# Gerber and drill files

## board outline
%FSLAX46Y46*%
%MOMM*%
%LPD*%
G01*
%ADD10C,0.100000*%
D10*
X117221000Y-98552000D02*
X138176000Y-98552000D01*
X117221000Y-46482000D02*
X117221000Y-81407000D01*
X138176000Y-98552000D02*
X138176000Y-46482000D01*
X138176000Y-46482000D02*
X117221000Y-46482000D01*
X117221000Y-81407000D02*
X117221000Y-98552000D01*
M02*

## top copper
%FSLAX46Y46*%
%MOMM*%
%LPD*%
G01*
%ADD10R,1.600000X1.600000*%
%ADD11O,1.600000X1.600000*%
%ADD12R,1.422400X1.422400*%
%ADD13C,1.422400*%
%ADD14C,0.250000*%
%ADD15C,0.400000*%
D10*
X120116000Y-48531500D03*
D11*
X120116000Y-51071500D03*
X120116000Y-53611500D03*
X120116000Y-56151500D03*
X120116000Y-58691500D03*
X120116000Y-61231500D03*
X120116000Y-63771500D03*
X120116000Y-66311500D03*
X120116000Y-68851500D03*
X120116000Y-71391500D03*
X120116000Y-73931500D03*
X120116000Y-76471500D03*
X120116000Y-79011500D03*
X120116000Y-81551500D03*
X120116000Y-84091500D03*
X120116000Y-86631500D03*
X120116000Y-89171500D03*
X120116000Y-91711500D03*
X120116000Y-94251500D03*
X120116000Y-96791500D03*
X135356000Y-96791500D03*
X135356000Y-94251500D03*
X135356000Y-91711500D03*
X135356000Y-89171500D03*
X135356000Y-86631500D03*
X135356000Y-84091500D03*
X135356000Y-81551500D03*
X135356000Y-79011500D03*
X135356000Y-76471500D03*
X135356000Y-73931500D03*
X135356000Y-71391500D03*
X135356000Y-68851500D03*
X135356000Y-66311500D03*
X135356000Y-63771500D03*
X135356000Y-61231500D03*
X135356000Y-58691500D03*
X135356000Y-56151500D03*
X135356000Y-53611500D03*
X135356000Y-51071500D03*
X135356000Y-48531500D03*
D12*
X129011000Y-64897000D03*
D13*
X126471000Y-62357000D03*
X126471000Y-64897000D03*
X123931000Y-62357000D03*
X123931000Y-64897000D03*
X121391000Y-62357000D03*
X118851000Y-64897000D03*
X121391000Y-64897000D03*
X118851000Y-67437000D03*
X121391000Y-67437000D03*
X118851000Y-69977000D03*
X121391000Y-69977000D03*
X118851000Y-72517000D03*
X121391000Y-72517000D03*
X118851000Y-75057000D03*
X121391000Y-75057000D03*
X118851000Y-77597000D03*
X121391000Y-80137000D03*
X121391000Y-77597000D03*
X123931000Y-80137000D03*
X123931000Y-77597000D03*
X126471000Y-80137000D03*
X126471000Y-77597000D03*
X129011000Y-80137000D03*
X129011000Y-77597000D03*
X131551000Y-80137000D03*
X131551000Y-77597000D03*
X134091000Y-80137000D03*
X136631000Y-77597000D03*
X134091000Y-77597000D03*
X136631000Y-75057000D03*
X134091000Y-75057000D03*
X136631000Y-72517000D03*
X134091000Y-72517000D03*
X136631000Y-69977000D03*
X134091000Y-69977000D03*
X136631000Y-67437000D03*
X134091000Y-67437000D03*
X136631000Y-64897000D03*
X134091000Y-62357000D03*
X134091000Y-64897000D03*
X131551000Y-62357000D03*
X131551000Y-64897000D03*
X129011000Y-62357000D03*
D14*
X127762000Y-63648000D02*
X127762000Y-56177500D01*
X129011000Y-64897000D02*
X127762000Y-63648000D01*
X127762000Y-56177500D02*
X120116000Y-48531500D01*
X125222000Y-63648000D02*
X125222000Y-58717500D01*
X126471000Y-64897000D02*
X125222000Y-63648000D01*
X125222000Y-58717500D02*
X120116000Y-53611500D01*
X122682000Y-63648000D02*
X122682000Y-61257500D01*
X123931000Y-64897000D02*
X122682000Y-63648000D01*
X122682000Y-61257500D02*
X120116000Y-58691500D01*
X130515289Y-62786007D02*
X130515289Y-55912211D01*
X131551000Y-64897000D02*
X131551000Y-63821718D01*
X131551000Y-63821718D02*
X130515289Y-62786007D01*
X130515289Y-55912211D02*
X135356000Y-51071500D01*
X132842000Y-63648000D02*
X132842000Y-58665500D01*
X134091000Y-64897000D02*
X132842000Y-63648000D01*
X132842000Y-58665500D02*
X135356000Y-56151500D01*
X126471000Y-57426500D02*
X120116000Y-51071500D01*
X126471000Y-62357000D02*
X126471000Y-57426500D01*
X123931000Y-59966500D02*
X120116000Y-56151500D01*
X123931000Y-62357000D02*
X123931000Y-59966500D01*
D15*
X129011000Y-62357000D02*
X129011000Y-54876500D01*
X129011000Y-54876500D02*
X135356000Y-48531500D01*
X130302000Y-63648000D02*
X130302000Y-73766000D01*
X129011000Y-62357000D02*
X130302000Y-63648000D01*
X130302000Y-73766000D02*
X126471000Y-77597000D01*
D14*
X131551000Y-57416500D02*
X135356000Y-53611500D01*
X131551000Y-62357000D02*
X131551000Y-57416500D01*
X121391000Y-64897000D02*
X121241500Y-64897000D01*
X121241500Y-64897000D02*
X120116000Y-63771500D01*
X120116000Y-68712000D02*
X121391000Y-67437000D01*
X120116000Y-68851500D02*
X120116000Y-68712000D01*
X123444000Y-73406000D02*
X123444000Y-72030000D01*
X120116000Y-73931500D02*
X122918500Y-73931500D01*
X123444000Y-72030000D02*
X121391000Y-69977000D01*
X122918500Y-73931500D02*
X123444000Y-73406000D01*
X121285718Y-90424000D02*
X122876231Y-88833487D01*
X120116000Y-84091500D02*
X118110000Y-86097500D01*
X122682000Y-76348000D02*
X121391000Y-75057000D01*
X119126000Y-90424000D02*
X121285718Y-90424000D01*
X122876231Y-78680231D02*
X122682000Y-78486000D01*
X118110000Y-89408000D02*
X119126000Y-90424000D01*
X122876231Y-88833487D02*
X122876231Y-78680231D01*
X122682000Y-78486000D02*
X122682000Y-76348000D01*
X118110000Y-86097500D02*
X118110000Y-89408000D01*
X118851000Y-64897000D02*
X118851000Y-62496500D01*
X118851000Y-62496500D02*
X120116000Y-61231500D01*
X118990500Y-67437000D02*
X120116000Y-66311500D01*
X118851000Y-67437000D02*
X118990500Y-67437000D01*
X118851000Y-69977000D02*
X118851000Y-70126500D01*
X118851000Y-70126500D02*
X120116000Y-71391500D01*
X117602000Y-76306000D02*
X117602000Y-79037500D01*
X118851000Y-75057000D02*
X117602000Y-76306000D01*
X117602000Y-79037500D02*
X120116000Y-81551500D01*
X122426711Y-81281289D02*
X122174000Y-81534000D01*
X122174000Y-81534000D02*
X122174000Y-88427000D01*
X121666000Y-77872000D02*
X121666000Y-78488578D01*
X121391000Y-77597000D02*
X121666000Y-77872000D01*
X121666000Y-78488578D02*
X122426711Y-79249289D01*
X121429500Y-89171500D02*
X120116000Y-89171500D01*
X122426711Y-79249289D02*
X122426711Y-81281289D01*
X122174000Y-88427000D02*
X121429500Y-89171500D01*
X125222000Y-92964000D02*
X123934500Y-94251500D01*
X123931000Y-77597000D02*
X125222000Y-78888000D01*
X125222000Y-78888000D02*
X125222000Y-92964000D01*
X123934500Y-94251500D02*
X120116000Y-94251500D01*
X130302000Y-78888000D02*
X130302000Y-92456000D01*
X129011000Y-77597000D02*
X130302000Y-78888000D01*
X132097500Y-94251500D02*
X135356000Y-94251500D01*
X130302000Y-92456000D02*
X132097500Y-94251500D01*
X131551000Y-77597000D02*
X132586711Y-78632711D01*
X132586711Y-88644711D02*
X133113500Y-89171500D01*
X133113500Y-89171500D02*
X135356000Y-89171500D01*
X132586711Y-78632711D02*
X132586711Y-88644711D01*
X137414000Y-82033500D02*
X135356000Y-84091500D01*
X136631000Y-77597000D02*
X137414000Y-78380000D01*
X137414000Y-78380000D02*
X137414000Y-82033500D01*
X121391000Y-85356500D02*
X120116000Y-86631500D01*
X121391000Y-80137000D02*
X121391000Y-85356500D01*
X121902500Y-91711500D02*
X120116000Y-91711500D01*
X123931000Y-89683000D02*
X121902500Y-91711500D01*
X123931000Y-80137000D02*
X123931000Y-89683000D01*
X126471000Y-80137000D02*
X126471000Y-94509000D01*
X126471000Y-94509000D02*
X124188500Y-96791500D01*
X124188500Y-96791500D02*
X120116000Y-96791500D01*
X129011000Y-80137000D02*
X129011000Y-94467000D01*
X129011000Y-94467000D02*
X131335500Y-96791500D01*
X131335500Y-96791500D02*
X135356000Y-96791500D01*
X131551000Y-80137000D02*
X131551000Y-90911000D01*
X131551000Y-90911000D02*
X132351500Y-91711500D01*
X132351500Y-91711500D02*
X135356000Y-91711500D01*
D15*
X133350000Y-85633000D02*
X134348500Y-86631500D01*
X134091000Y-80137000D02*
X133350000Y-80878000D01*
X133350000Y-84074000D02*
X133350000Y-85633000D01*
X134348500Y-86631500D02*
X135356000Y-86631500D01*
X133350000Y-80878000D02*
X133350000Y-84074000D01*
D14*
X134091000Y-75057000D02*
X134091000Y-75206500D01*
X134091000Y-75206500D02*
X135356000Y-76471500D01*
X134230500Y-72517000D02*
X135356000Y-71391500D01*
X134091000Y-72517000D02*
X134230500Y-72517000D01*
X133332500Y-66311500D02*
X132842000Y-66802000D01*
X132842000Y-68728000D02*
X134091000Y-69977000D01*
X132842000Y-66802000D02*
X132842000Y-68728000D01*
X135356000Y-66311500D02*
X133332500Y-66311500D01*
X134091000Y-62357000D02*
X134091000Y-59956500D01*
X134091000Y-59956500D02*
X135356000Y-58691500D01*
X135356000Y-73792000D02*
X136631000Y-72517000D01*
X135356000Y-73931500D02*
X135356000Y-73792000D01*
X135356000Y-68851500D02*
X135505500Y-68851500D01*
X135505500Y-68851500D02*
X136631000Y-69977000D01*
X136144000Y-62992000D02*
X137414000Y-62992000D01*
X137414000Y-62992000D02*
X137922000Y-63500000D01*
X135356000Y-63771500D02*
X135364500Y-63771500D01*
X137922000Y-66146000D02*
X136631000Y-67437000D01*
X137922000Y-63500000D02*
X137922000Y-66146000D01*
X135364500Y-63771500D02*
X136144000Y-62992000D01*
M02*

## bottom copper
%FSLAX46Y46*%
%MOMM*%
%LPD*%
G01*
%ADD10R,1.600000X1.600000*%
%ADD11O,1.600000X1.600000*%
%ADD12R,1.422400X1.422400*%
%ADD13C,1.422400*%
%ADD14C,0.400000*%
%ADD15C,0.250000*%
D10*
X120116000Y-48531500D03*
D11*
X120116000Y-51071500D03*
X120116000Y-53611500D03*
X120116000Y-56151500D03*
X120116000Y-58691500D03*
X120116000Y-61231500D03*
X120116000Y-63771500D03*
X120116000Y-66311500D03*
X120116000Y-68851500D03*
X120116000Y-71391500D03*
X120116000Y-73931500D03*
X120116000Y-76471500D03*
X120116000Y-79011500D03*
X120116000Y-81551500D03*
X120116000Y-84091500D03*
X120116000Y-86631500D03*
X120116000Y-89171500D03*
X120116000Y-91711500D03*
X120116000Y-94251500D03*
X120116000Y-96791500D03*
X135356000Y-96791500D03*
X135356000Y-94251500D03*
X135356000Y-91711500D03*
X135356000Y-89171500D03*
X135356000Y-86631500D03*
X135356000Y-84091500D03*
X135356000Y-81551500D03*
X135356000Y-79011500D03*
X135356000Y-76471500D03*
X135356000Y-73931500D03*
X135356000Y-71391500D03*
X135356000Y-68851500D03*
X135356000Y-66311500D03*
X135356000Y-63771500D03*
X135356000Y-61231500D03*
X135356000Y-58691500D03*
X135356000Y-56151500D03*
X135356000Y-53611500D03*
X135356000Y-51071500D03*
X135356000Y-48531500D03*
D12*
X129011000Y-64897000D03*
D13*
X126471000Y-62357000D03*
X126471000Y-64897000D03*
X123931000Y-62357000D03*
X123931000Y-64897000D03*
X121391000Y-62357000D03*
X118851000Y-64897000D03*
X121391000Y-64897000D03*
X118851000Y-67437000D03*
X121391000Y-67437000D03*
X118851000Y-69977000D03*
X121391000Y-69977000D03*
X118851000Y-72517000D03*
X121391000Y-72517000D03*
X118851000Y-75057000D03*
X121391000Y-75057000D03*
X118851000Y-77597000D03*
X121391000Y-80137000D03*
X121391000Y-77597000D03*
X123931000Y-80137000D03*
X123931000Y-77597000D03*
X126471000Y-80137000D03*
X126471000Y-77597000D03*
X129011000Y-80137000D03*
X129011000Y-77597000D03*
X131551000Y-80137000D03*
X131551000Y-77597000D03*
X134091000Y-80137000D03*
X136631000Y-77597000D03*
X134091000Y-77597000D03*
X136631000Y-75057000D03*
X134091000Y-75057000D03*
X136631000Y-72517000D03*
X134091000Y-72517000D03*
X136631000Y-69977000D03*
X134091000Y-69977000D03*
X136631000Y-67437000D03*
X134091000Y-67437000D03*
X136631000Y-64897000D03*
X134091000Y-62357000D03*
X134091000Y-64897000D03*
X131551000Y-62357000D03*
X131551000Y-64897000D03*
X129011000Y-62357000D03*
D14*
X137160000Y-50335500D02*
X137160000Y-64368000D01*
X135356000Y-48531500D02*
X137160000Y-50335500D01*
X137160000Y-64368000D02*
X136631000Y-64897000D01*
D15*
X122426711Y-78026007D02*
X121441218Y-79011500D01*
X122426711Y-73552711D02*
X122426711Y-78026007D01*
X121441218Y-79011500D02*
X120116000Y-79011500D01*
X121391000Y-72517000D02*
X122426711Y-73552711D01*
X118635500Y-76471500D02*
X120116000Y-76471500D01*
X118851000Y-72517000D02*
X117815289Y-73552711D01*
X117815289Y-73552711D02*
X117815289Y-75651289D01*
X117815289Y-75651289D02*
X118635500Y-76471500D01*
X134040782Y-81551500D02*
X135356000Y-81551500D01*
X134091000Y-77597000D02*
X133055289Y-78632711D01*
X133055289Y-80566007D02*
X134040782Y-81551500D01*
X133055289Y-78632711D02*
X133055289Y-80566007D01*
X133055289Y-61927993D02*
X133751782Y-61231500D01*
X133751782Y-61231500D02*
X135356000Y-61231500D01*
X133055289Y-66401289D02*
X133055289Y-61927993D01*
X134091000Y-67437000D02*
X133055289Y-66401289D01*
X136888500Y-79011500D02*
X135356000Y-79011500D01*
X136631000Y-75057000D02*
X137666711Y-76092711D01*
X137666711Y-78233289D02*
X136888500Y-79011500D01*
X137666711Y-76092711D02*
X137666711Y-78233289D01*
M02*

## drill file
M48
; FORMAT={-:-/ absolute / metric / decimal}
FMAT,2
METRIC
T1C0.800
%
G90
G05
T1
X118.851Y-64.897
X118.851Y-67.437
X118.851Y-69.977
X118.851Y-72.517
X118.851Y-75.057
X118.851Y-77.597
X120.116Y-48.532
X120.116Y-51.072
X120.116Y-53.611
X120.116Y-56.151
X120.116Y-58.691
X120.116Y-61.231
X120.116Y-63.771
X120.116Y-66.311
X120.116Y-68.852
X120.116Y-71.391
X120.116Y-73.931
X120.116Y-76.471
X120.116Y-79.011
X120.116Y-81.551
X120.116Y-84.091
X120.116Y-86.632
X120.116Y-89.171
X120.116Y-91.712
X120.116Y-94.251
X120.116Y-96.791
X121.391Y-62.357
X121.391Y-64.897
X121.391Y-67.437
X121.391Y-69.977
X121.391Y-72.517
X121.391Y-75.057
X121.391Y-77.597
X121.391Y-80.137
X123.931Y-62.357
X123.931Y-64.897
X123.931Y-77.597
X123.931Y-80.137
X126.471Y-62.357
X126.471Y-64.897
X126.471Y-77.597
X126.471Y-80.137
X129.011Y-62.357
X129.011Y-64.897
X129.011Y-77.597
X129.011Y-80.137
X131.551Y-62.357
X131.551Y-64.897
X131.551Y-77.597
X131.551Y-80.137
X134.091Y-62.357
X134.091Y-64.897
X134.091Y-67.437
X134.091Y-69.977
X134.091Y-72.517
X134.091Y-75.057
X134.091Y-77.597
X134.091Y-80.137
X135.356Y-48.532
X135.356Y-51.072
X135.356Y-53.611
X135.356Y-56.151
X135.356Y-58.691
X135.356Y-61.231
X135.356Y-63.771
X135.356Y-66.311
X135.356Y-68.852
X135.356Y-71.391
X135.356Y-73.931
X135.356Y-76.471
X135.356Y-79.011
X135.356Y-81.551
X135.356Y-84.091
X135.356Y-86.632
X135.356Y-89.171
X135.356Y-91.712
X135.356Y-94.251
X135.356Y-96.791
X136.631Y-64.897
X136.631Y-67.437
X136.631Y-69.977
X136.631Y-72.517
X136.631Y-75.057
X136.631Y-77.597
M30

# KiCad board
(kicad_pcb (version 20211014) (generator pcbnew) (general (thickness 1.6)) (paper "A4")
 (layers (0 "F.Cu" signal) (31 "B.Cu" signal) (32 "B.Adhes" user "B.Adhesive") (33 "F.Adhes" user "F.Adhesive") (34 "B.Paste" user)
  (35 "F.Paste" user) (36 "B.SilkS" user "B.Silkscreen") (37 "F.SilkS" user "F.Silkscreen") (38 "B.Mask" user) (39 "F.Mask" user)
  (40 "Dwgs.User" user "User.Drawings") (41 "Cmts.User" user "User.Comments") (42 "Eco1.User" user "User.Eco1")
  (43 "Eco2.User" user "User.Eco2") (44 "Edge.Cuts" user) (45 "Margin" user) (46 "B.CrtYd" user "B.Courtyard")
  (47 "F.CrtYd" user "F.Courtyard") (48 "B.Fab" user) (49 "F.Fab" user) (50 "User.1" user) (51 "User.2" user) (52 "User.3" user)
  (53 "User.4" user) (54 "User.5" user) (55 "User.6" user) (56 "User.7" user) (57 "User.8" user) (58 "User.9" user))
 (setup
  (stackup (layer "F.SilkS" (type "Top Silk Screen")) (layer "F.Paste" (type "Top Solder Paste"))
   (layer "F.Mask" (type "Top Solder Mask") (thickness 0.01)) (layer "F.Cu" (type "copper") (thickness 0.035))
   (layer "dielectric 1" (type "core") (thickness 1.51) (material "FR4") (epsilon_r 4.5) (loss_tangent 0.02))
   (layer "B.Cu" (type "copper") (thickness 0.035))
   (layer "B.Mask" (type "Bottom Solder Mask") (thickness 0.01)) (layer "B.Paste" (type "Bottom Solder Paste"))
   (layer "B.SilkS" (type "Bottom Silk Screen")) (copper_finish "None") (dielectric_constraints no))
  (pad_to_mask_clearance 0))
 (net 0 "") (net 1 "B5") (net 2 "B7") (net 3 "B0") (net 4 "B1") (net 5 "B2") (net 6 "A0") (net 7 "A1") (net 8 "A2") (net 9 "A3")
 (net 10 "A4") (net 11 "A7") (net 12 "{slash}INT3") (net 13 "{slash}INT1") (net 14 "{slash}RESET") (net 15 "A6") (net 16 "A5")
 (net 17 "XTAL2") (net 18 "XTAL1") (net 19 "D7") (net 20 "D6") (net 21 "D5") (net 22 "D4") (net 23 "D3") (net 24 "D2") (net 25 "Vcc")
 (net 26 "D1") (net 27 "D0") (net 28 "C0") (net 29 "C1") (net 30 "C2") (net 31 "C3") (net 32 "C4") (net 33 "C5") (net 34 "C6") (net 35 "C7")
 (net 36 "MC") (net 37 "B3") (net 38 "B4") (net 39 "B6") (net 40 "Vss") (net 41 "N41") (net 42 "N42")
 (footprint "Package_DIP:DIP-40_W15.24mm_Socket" (layer "F.Cu") (at 120.116 48.5315)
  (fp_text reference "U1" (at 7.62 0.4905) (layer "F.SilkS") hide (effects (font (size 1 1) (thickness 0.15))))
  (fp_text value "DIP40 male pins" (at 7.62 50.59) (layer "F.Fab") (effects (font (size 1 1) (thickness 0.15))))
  (pad "1" thru_hole rect locked (at 0 0) (size 1.6 1.6) (drill 0.8) (layers *.Cu *.Mask) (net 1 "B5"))
  (pad "2" thru_hole oval locked (at 0 2.54) (size 1.6 1.6) (drill 0.8) (layers *.Cu *.Mask) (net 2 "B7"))
  (pad "3" thru_hole oval locked (at 0 5.08) (size 1.6 1.6) (drill 0.8) (layers *.Cu *.Mask) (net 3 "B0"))
  (pad "4" thru_hole oval locked (at 0 7.62) (size 1.6 1.6) (drill 0.8) (layers *.Cu *.Mask) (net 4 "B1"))
  (pad "5" thru_hole oval locked (at 0 10.16) (size 1.6 1.6) (drill 0.8) (layers *.Cu *.Mask) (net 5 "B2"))
  (pad "6" thru_hole oval locked (at 0 12.7) (size 1.6 1.6) (drill 0.8) (layers *.Cu *.Mask) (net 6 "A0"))
  (pad "7" thru_hole oval locked (at 0 15.24) (size 1.6 1.6) (drill 0.8) (layers *.Cu *.Mask) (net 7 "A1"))
  (pad "8" thru_hole oval locked (at 0 17.78) (size 1.6 1.6) (drill 0.8) (layers *.Cu *.Mask) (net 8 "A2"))
  (pad "9" thru_hole oval locked (at 0 20.32) (size 1.6 1.6) (drill 0.8) (layers *.Cu *.Mask) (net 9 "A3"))
  (pad "10" thru_hole oval locked (at 0 22.86) (size 1.6 1.6) (drill 0.8) (layers *.Cu *.Mask) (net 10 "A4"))
  (pad "11" thru_hole oval locked (at 0 25.4) (size 1.6 1.6) (drill 0.8) (layers *.Cu *.Mask) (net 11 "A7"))
  (pad "12" thru_hole oval locked (at 0 27.94) (size 1.6 1.6) (drill 0.8) (layers *.Cu *.Mask) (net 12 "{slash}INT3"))
  (pad "13" thru_hole oval locked (at 0 30.48) (size 1.6 1.6) (drill 0.8) (layers *.Cu *.Mask) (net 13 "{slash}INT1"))
  (pad "14" thru_hole oval locked (at 0 33.02) (size 1.6 1.6) (drill 0.8) (layers *.Cu *.Mask) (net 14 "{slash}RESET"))
  (pad "15" thru_hole oval locked (at 0 35.56) (size 1.6 1.6) (drill 0.8) (layers *.Cu *.Mask) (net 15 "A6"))
  (pad "16" thru_hole oval locked (at 0 38.1) (size 1.6 1.6) (drill 0.8) (layers *.Cu *.Mask) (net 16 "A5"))
  (pad "17" thru_hole oval locked (at 0 40.64) (size 1.6 1.6) (drill 0.8) (layers *.Cu *.Mask) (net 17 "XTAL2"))
  (pad "18" thru_hole oval locked (at 0 43.18) (size 1.6 1.6) (drill 0.8) (layers *.Cu *.Mask) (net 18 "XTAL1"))
  (pad "19" thru_hole oval locked (at 0 45.72) (size 1.6 1.6) (drill 0.8) (layers *.Cu *.Mask) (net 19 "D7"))
  (pad "20" thru_hole oval locked (at 0 48.26) (size 1.6 1.6) (drill 0.8) (layers *.Cu *.Mask) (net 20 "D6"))
  (pad "21" thru_hole oval locked (at 15.24 48.26) (size 1.6 1.6) (drill 0.8) (layers *.Cu *.Mask) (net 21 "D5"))
  (pad "22" thru_hole oval locked (at 15.24 45.72) (size 1.6 1.6) (drill 0.8) (layers *.Cu *.Mask) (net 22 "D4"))
  (pad "23" thru_hole oval locked (at 15.24 43.18) (size 1.6 1.6) (drill 0.8) (layers *.Cu *.Mask) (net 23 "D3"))
  (pad "24" thru_hole oval locked (at 15.24 40.64) (size 1.6 1.6) (drill 0.8) (layers *.Cu *.Mask) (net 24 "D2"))
  (pad "25" thru_hole oval locked (at 15.24 38.1) (size 1.6 1.6) (drill 0.8) (layers *.Cu *.Mask) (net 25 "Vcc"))
  (pad "26" thru_hole oval locked (at 15.24 35.56) (size 1.6 1.6) (drill 0.8) (layers *.Cu *.Mask) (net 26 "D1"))
  (pad "27" thru_hole oval locked (at 15.24 33.02) (size 1.6 1.6) (drill 0.8) (layers *.Cu *.Mask) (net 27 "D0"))
  (pad "28" thru_hole oval locked (at 15.24 30.48) (size 1.6 1.6) (drill 0.8) (layers *.Cu *.Mask) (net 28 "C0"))
  (pad "29" thru_hole oval locked (at 15.24 27.94) (size 1.6 1.6) (drill 0.8) (layers *.Cu *.Mask) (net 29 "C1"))
  (pad "30" thru_hole oval locked (at 15.24 25.4) (size 1.6 1.6) (drill 0.8) (layers *.Cu *.Mask) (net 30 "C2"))
  (pad "31" thru_hole oval locked (at 15.24 22.86) (size 1.6 1.6) (drill 0.8) (layers *.Cu *.Mask) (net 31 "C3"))
  (pad "32" thru_hole oval locked (at 15.24 20.32) (size 1.6 1.6) (drill 0.8) (layers *.Cu *.Mask) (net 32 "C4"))
  (pad "33" thru_hole oval locked (at 15.24 17.78) (size 1.6 1.6) (drill 0.8) (layers *.Cu *.Mask) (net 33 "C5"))
  (pad "34" thru_hole oval locked (at 15.24 15.24) (size 1.6 1.6) (drill 0.8) (layers *.Cu *.Mask) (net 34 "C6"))
  (pad "35" thru_hole oval locked (at 15.24 12.7) (size 1.6 1.6) (drill 0.8) (layers *.Cu *.Mask) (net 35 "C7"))
  (pad "36" thru_hole oval locked (at 15.24 10.16) (size 1.6 1.6) (drill 0.8) (layers *.Cu *.Mask) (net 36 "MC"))
  (pad "37" thru_hole oval locked (at 15.24 7.62) (size 1.6 1.6) (drill 0.8) (layers *.Cu *.Mask) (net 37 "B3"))
  (pad "38" thru_hole oval locked (at 15.24 5.08) (size 1.6 1.6) (drill 0.8) (layers *.Cu *.Mask) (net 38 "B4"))
  (pad "39" thru_hole oval locked (at 15.24 2.54) (size 1.6 1.6) (drill 0.8) (layers *.Cu *.Mask) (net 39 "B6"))
  (pad "40" thru_hole oval locked (at 15.24 0) (size 1.6 1.6) (drill 0.8) (layers *.Cu *.Mask) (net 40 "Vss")))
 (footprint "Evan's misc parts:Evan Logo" (layer "F.Cu") (at 127.381 91.567)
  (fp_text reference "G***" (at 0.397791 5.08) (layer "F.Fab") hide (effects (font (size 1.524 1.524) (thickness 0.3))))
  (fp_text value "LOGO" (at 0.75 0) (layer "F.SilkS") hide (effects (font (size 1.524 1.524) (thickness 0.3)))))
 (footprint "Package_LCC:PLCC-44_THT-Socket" (layer "F.Cu") (at 129.011 64.897)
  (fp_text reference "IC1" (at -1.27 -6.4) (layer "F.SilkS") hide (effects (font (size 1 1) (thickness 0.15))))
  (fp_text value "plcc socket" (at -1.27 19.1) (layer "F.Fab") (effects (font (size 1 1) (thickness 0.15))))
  (pad "1" thru_hole rect locked (at 0 0) (size 1.4224 1.4224) (drill 0.8) (layers *.Cu *.Mask) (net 1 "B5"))
  (pad "2" thru_hole circle locked (at -2.54 -2.54) (size 1.4224 1.4224) (drill 0.8) (layers *.Cu *.Mask) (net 2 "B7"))
  (pad "3" thru_hole circle locked (at -2.54 0) (size 1.4224 1.4224) (drill 0.8) (layers *.Cu *.Mask) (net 3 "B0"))
  (pad "4" thru_hole circle locked (at -5.08 -2.54) (size 1.4224 1.4224) (drill 0.8) (layers *.Cu *.Mask) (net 4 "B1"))
  (pad "5" thru_hole circle locked (at -5.08 0) (size 1.4224 1.4224) (drill 0.8) (layers *.Cu *.Mask) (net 5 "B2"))
  (pad "6" thru_hole circle locked (at -7.62 -2.54) (size 1.4224 1.4224) (drill 0.8) (layers *.Cu *.Mask) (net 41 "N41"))
  (pad "7" thru_hole circle locked (at -10.16 0) (size 1.4224 1.4224) (drill 0.8) (layers *.Cu *.Mask) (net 6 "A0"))
  (pad "8" thru_hole circle locked (at -7.62 0) (size 1.4224 1.4224) (drill 0.8) (layers *.Cu *.Mask) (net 7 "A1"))
  (pad "9" thru_hole circle locked (at -10.16 2.54) (size 1.4224 1.4224) (drill 0.8) (layers *.Cu *.Mask) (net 8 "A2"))
  (pad "10" thru_hole circle locked (at -7.62 2.54) (size 1.4224 1.4224) (drill 0.8) (layers *.Cu *.Mask) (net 9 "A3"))
  (pad "11" thru_hole circle locked (at -10.16 5.08) (size 1.4224 1.4224) (drill 0.8) (layers *.Cu *.Mask) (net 10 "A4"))
  (pad "12" thru_hole circle locked (at -7.62 5.08) (size 1.4224 1.4224) (drill 0.8) (layers *.Cu *.Mask) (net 11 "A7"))
  (pad "13" thru_hole circle locked (at -10.16 7.62) (size 1.4224 1.4224) (drill 0.8) (layers *.Cu *.Mask) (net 12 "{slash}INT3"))
  (pad "14" thru_hole circle locked (at -7.62 7.62) (size 1.4224 1.4224) (drill 0.8) (layers *.Cu *.Mask) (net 13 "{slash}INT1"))
  (pad "15" thru_hole circle locked (at -10.16 10.16) (size 1.4224 1.4224) (drill 0.8) (layers *.Cu *.Mask) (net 14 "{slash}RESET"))
  (pad "16" thru_hole circle locked (at -7.62 10.16) (size 1.4224 1.4224) (drill 0.8) (layers *.Cu *.Mask) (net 15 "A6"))
  (pad "17" thru_hole circle locked (at -10.16 12.7) (size 1.4224 1.4224) (drill 0.8) (layers *.Cu *.Mask) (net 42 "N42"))
  (pad "18" thru_hole circle locked (at -7.62 15.24) (size 1.4224 1.4224) (drill 0.8) (layers *.Cu *.Mask) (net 16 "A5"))
  (pad "19" thru_hole circle locked (at -7.62 12.7) (size 1.4224 1.4224) (drill 0.8) (layers *.Cu *.Mask) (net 17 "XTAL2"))
  (pad "20" thru_hole circle locked (at -5.08 15.24) (size 1.4224 1.4224) (drill 0.8) (layers *.Cu *.Mask) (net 18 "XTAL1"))
  (pad "21" thru_hole circle locked (at -5.08 12.7) (size 1.4224 1.4224) (drill 0.8) (layers *.Cu *.Mask) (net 19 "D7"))
  (pad "22" thru_hole circle locked (at -2.54 15.24) (size 1.4224 1.4224) (drill 0.8) (layers *.Cu *.Mask) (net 20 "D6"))
  (pad "23" thru_hole circle locked (at -2.54 12.7) (size 1.4224 1.4224) (drill 0.8) (layers *.Cu *.Mask) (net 40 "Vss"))
  (pad "24" thru_hole circle locked (at 0 15.24) (size 1.4224 1.4224) (drill 0.8) (layers *.Cu *.Mask) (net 21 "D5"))
  (pad "25" thru_hole circle locked (at 0 12.7) (size 1.4224 1.4224) (drill 0.8) (layers *.Cu *.Mask) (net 22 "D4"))
  (pad "26" thru_hole circle locked (at 2.54 15.24) (size 1.4224 1.4224) (drill 0.8) (layers *.Cu *.Mask) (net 23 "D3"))
  (pad "27" thru_hole circle locked (at 2.54 12.7) (size 1.4224 1.4224) (drill 0.8) (layers *.Cu *.Mask) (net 24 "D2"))
  (pad "28" thru_hole circle locked (at 5.08 15.24) (size 1.4224 1.4224) (drill 0.8) (layers *.Cu *.Mask) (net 25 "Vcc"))
  (pad "29" thru_hole circle locked (at 7.62 12.7) (size 1.4224 1.4224) (drill 0.8) (layers *.Cu *.Mask) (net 26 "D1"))
  (pad "30" thru_hole circle locked (at 5.08 12.7) (size 1.4224 1.4224) (drill 0.8) (layers *.Cu *.Mask) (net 27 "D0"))
  (pad "31" thru_hole circle locked (at 7.62 10.16) (size 1.4224 1.4224) (drill 0.8) (layers *.Cu *.Mask) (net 28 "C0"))
  (pad "32" thru_hole circle locked (at 5.08 10.16) (size 1.4224 1.4224) (drill 0.8) (layers *.Cu *.Mask) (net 29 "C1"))
  (pad "33" thru_hole circle locked (at 7.62 7.62) (size 1.4224 1.4224) (drill 0.8) (layers *.Cu *.Mask) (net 30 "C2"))
  (pad "34" thru_hole circle locked (at 5.08 7.62) (size 1.4224 1.4224) (drill 0.8) (layers *.Cu *.Mask) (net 31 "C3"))
  (pad "35" thru_hole circle locked (at 7.62 5.08) (size 1.4224 1.4224) (drill 0.8) (layers *.Cu *.Mask) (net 32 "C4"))
  (pad "36" thru_hole circle locked (at 5.08 5.08) (size 1.4224 1.4224) (drill 0.8) (layers *.Cu *.Mask) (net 33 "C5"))
  (pad "37" thru_hole circle locked (at 7.62 2.54) (size 1.4224 1.4224) (drill 0.8) (layers *.Cu *.Mask) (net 34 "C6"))
  (pad "38" thru_hole circle locked (at 5.08 2.54) (size 1.4224 1.4224) (drill 0.8) (layers *.Cu *.Mask) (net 35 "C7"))
  (pad "39" thru_hole circle locked (at 7.62 0) (size 1.4224 1.4224) (drill 0.8) (layers *.Cu *.Mask) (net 40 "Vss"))
  (pad "40" thru_hole circle locked (at 5.08 -2.54) (size 1.4224 1.4224) (drill 0.8) (layers *.Cu *.Mask) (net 36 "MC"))
  (pad "41" thru_hole circle locked (at 5.08 0) (size 1.4224 1.4224) (drill 0.8) (layers *.Cu *.Mask) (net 37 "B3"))
  (pad "42" thru_hole circle locked (at 2.54 -2.54) (size 1.4224 1.4224) (drill 0.8) (layers *.Cu *.Mask) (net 38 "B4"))
  (pad "43" thru_hole circle locked (at 2.54 0) (size 1.4224 1.4224) (drill 0.8) (layers *.Cu *.Mask) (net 39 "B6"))
  (pad "44" thru_hole circle locked (at 0 -2.54) (size 1.4224 1.4224) (drill 0.8) (layers *.Cu *.Mask) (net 40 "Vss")))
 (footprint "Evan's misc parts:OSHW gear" (layer "B.Cu") (at 127.381 90.932 180)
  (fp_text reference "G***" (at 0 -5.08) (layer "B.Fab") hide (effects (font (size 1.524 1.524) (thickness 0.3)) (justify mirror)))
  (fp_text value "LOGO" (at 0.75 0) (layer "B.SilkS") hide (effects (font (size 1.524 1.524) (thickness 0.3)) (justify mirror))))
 (gr_line (start 117.221 98.552) (end 138.176 98.552) (layer "Edge.Cuts") (width 0.1))
 (gr_line (start 117.221 46.482) (end 117.221 81.407) (layer "Edge.Cuts") (width 0.1))
 (gr_line (start 138.176 98.552) (end 138.176 46.482) (layer "Edge.Cuts") (width 0.1))
 (gr_line (start 138.176 46.482) (end 117.221 46.482) (layer "Edge.Cuts") (width 0.1))
 (gr_line (start 117.221 81.407) (end 117.221 98.552) (layer "Edge.Cuts") (width 0.1))
 (segment (start 127.762 63.648) (end 127.762 56.1775) (width 0.25) (layer "F.Cu") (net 1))
 (segment (start 129.011 64.897) (end 127.762 63.648) (width 0.25) (layer "F.Cu") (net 1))
 (segment (start 127.762 56.1775) (end 120.116 48.5315) (width 0.25) (layer "F.Cu") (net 1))
 (segment (start 125.222 63.648) (end 125.222 58.7175) (width 0.25) (layer "F.Cu") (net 3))
 (segment (start 126.471 64.897) (end 125.222 63.648) (width 0.25) (layer "F.Cu") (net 3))
 (segment (start 125.222 58.7175) (end 120.116 53.6115) (width 0.25) (layer "F.Cu") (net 3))
 (segment (start 122.682 63.648) (end 122.682 61.2575) (width 0.25) (layer "F.Cu") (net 5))
 (segment (start 123.931 64.897) (end 122.682 63.648) (width 0.25) (layer "F.Cu") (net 5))
 (segment (start 122.682 61.2575) (end 120.116 58.6915) (width 0.25) (layer "F.Cu") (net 5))
 (segment (start 130.515289 62.786007) (end 130.515289 55.912211) (width 0.25) (layer "F.Cu") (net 39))
 (segment (start 131.551 64.897) (end 131.551 63.821718) (width 0.25) (layer "F.Cu") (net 39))
 (segment (start 131.551 63.821718) (end 130.515289 62.786007) (width 0.25) (layer "F.Cu") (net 39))
 (segment (start 130.515289 55.912211) (end 135.356 51.0715) (width 0.25) (layer "F.Cu") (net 39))
 (segment (start 132.842 63.648) (end 132.842 58.6655) (width 0.25) (layer "F.Cu") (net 37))
 (segment (start 134.091 64.897) (end 132.842 63.648) (width 0.25) (layer "F.Cu") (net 37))
 (segment (start 132.842 58.6655) (end 135.356 56.1515) (width 0.25) (layer "F.Cu") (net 37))
 (segment (start 126.471 57.4265) (end 120.116 51.0715) (width 0.25) (layer "F.Cu") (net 2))
 (segment (start 126.471 62.357) (end 126.471 57.4265) (width 0.25) (layer "F.Cu") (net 2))
 (segment (start 123.931 59.9665) (end 120.116 56.1515) (width 0.25) (layer "F.Cu") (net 4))
 (segment (start 123.931 62.357) (end 123.931 59.9665) (width 0.25) (layer "F.Cu") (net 4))
 (segment (start 129.011 62.357) (end 129.011 54.8765) (width 0.4) (layer "F.Cu") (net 40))
 (segment (start 129.011 54.8765) (end 135.356 48.5315) (width 0.4) (layer "F.Cu") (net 40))
 (segment (start 130.302 63.648) (end 130.302 73.766) (width 0.4) (layer "F.Cu") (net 40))
 (segment (start 129.011 62.357) (end 130.302 63.648) (width 0.4) (layer "F.Cu") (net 40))
 (segment (start 130.302 73.766) (end 126.471 77.597) (width 0.4) (layer "F.Cu") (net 40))
 (segment (start 137.16 50.3355) (end 137.16 64.368) (width 0.4) (layer "B.Cu") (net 40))
 (segment (start 135.356 48.5315) (end 137.16 50.3355) (width 0.4) (layer "B.Cu") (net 40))
 (segment (start 137.16 64.368) (end 136.631 64.897) (width 0.4) (layer "B.Cu") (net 40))
 (segment (start 131.551 57.4165) (end 135.356 53.6115) (width 0.25) (layer "F.Cu") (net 38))
 (segment (start 131.551 62.357) (end 131.551 57.4165) (width 0.25) (layer "F.Cu") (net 38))
 (segment (start 121.391 64.897) (end 121.2415 64.897) (width 0.25) (layer "F.Cu") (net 7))
 (segment (start 121.2415 64.897) (end 120.116 63.7715) (width 0.25) (layer "F.Cu") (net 7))
 (segment (start 120.116 68.712) (end 121.391 67.437) (width 0.25) (layer "F.Cu") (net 9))
 (segment (start 120.116 68.8515) (end 120.116 68.712) (width 0.25) (layer "F.Cu") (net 9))
 (segment (start 123.444 73.406) (end 123.444 72.03) (width 0.25) (layer "F.Cu") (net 11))
 (segment (start 120.116 73.9315) (end 122.9185 73.9315) (width 0.25) (layer "F.Cu") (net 11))
 (segment (start 123.444 72.03) (end 121.391 69.977) (width 0.25) (layer "F.Cu") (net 11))
 (segment (start 122.9185 73.9315) (end 123.444 73.406) (width 0.25) (layer "F.Cu") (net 11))
 (segment (start 122.426711 78.026007) (end 121.441218 79.0115) (width 0.25) (layer "B.Cu") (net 13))
 (segment (start 122.426711 73.552711) (end 122.426711 78.026007) (width 0.25) (layer "B.Cu") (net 13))
 (segment (start 121.441218 79.0115) (end 120.116 79.0115) (width 0.25) (layer "B.Cu") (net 13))
 (segment (start 121.391 72.517) (end 122.426711 73.552711) (width 0.25) (layer "B.Cu") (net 13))
 (segment (start 121.285718 90.424) (end 122.876231 88.833487) (width 0.25) (layer "F.Cu") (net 15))
 (segment (start 120.116 84.0915) (end 118.11 86.0975) (width 0.25) (layer "F.Cu") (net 15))
 (segment (start 122.682 76.348) (end 121.391 75.057) (width 0.25) (layer "F.Cu") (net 15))
 (segment (start 119.126 90.424) (end 121.285718 90.424) (width 0.25) (layer "F.Cu") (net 15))
 (segment (start 122.876231 78.680231) (end 122.682 78.486) (width 0.25) (layer "F.Cu") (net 15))
 (segment (start 118.11 89.408) (end 119.126 90.424) (width 0.25) (layer "F.Cu") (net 15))
 (segment (start 122.876231 88.833487) (end 122.876231 78.680231) (width 0.25) (layer "F.Cu") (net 15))
 (segment (start 122.682 78.486) (end 122.682 76.348) (width 0.25) (layer "F.Cu") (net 15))
 (segment (start 118.11 86.0975) (end 118.11 89.408) (width 0.25) (layer "F.Cu") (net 15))
 (segment (start 118.851 64.897) (end 118.851 62.4965) (width 0.25) (layer "F.Cu") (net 6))
 (segment (start 118.851 62.4965) (end 120.116 61.2315) (width 0.25) (layer "F.Cu") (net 6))
 (segment (start 118.9905 67.437) (end 120.116 66.3115) (width 0.25) (layer "F.Cu") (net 8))
 (segment (start 118.851 67.437) (end 118.9905 67.437) (width 0.25) (layer "F.Cu") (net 8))
 (segment (start 118.851 69.977) (end 118.851 70.1265) (width 0.25) (layer "F.Cu") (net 10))
 (segment (start 118.851 70.1265) (end 120.116 71.3915) (width 0.25) (layer "F.Cu") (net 10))
 (segment (start 118.6355 76.4715) (end 120.116 76.4715) (width 0.25) (layer "B.Cu") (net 12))
 (segment (start 118.851 72.517) (end 117.815289 73.552711) (width 0.25) (layer "B.Cu") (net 12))
 (segment (start 117.815289 73.552711) (end 117.815289 75.651289) (width 0.25) (layer "B.Cu") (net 12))
 (segment (start 117.815289 75.651289) (end 118.6355 76.4715) (width 0.25) (layer "B.Cu") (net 12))
 (segment (start 117.602 76.306) (end 117.602 79.0375) (width 0.25) (layer "F.Cu") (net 14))
 (segment (start 118.851 75.057) (end 117.602 76.306) (width 0.25) (layer "F.Cu") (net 14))
 (segment (start 117.602 79.0375) (end 120.116 81.5515) (width 0.25) (layer "F.Cu") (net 14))
 (segment (start 122.426711 81.281289) (end 122.174 81.534) (width 0.25) (layer "F.Cu") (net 17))
 (segment (start 122.174 81.534) (end 122.174 88.427) (width 0.25) (layer "F.Cu") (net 17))
 (segment (start 121.666 77.872) (end 121.666 78.488578) (width 0.25) (layer "F.Cu") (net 17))
 (segment (start 121.391 77.597) (end 121.666 77.872) (width 0.25) (layer "F.Cu") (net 17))
 (segment (start 121.666 78.488578) (end 122.426711 79.249289) (width 0.25) (layer "F.Cu") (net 17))
 (segment (start 121.4295 89.1715) (end 120.116 89.1715) (width 0.25) (layer "F.Cu") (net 17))
 (segment (start 122.426711 79.249289) (end 122.426711 81.281289) (width 0.25) (layer "F.Cu") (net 17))
 (segment (start 122.174 88.427) (end 121.4295 89.1715) (width 0.25) (layer "F.Cu") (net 17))
 (segment (start 125.222 92.964) (end 123.9345 94.2515) (width 0.25) (layer "F.Cu") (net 19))
 (segment (start 123.931 77.597) (end 125.222 78.888) (width 0.25) (layer "F.Cu") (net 19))
 (segment (start 125.222 78.888) (end 125.222 92.964) (width 0.25) (layer "F.Cu") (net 19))
 (segment (start 123.9345 94.2515) (end 120.116 94.2515) (width 0.25) (layer "F.Cu") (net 19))
 (segment (start 130.302 78.888) (end 130.302 92.456) (width 0.25) (layer "F.Cu") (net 22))
 (segment (start 129.011 77.597) (end 130.302 78.888) (width 0.25) (layer "F.Cu") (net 22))
 (segment (start 132.0975 94.2515) (end 135.356 94.2515) (width 0.25) (layer "F.Cu") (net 22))
 (segment (start 130.302 92.456) (end 132.0975 94.2515) (width 0.25) (layer "F.Cu") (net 22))
 (segment (start 131.551 77.597) (end 132.586711 78.632711) (width 0.25) (layer "F.Cu") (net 24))
 (segment (start 132.586711 88.644711) (end 133.1135 89.1715) (width 0.25) (layer "F.Cu") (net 24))
 (segment (start 133.1135 89.1715) (end 135.356 89.1715) (width 0.25) (layer "F.Cu") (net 24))
 (segment (start 132.586711 78.632711) (end 132.586711 88.644711) (width 0.25) (layer "F.Cu") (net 24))
 (segment (start 137.414 82.0335) (end 135.356 84.0915) (width 0.25) (layer "F.Cu") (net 26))
 (segment (start 136.631 77.597) (end 137.414 78.38) (width 0.25) (layer "F.Cu") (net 26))
 (segment (start 137.414 78.38) (end 137.414 82.0335) (width 0.25) (layer "F.Cu") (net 26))
 (segment (start 121.391 85.3565) (end 120.116 86.6315) (width 0.25) (layer "F.Cu") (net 16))
 (segment (start 121.391 80.137) (end 121.391 85.3565) (width 0.25) (layer "F.Cu") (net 16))
 (segment (start 121.9025 91.7115) (end 120.116 91.7115) (width 0.25) (layer "F.Cu") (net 18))
 (segment (start 123.931 89.683) (end 121.9025 91.7115) (width 0.25) (layer "F.Cu") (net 18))
 (segment (start 123.931 80.137) (end 123.931 89.683) (width 0.25) (layer "F.Cu") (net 18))
 (segment (start 126.471 80.137) (end 126.471 94.509) (width 0.25) (layer "F.Cu") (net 20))
 (segment (start 126.471 94.509) (end 124.1885 96.7915) (width 0.25) (layer "F.Cu") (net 20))
 (segment (start 124.1885 96.7915) (end 120.116 96.7915) (width 0.25) (layer "F.Cu") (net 20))
 (segment (start 129.011 80.137) (end 129.011 94.467) (width 0.25) (layer "F.Cu") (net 21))
 (segment (start 129.011 94.467) (end 131.3355 96.7915) (width 0.25) (layer "F.Cu") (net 21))
 (segment (start 131.3355 96.7915) (end 135.356 96.7915) (width 0.25) (layer "F.Cu") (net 21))
 (segment (start 131.551 80.137) (end 131.551 90.911) (width 0.25) (layer "F.Cu") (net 23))
 (segment (start 131.551 90.911) (end 132.3515 91.7115) (width 0.25) (layer "F.Cu") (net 23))
 (segment (start 132.3515 91.7115) (end 135.356 91.7115) (width 0.25) (layer "F.Cu") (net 23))
 (segment (start 133.35 85.633) (end 134.3485 86.6315) (width 0.4) (layer "F.Cu") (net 25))
 (segment (start 134.091 80.137) (end 133.35 80.878) (width 0.4) (layer "F.Cu") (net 25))
 (segment (start 133.35 84.074) (end 133.35 85.633) (width 0.4) (layer "F.Cu") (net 25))
 (segment (start 134.3485 86.6315) (end 135.356 86.6315) (width 0.4) (layer "F.Cu") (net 25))
 (segment (start 133.35 80.878) (end 133.35 84.074) (width 0.4) (layer "F.Cu") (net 25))
 (segment (start 134.040782 81.5515) (end 135.356 81.5515) (width 0.25) (layer "B.Cu") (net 27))
 (segment (start 134.091 77.597) (end 133.055289 78.632711) (width 0.25) (layer "B.Cu") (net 27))
 (segment (start 133.055289 80.566007) (end 134.040782 81.5515) (width 0.25) (layer "B.Cu") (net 27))
 (segment (start 133.055289 78.632711) (end 133.055289 80.566007) (width 0.25) (layer "B.Cu") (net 27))
 (segment (start 134.091 75.057) (end 134.091 75.2065) (width 0.25) (layer "F.Cu") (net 29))
 (segment (start 134.091 75.2065) (end 135.356 76.4715) (width 0.25) (layer "F.Cu") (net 29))
 (segment (start 134.2305 72.517) (end 135.356 71.3915) (width 0.25) (layer "F.Cu") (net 31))
 (segment (start 134.091 72.517) (end 134.2305 72.517) (width 0.25) (layer "F.Cu") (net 31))
 (segment (start 133.3325 66.3115) (end 132.842 66.802) (width 0.25) (layer "F.Cu") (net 33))
 (segment (start 132.842 68.728) (end 134.091 69.977) (width 0.25) (layer "F.Cu") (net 33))
 (segment (start 132.842 66.802) (end 132.842 68.728) (width 0.25) (layer "F.Cu") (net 33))
 (segment (start 135.356 66.3115) (end 133.3325 66.3115) (width 0.25) (layer "F.Cu") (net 33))
 (segment (start 133.055289 61.927993) (end 133.751782 61.2315) (width 0.25) (layer "B.Cu") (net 35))
 (segment (start 133.751782 61.2315) (end 135.356 61.2315) (width 0.25) (layer "B.Cu") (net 35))
 (segment (start 133.055289 66.401289) (end 133.055289 61.927993) (width 0.25) (layer "B.Cu") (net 35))
 (segment (start 134.091 67.437) (end 133.055289 66.401289) (width 0.25) (layer "B.Cu") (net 35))
 (segment (start 134.091 62.357) (end 134.091 59.9565) (width 0.25) (layer "F.Cu") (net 36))
 (segment (start 134.091 59.9565) (end 135.356 58.6915) (width 0.25) (layer "F.Cu") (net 36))
 (segment (start 136.8885 79.0115) (end 135.356 79.0115) (width 0.25) (layer "B.Cu") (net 28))
 (segment (start 136.631 75.057) (end 137.666711 76.092711) (width 0.25) (layer "B.Cu") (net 28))
 (segment (start 137.666711 78.233289) (end 136.8885 79.0115) (width 0.25) (layer "B.Cu") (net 28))
 (segment (start 137.666711 76.092711) (end 137.666711 78.233289) (width 0.25) (layer "B.Cu") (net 28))
 (segment (start 135.356 73.792) (end 136.631 72.517) (width 0.25) (layer "F.Cu") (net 30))
 (segment (start 135.356 73.9315) (end 135.356 73.792) (width 0.25) (layer "F.Cu") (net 30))
 (segment (start 135.356 68.8515) (end 135.5055 68.8515) (width 0.25) (layer "F.Cu") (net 32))
 (segment (start 135.5055 68.8515) (end 136.631 69.977) (width 0.25) (layer "F.Cu") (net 32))
 (segment (start 136.144 62.992) (end 137.414 62.992) (width 0.25) (layer "F.Cu") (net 34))
 (segment (start 137.414 62.992) (end 137.922 63.5) (width 0.25) (layer "F.Cu") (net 34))
 (segment (start 135.356 63.7715) (end 135.3645 63.7715) (width 0.25) (layer "F.Cu") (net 34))
 (segment (start 137.922 66.146) (end 136.631 67.437) (width 0.25) (layer "F.Cu") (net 34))
 (segment (start 137.922 63.5) (end 137.922 66.146) (width 0.25) (layer "F.Cu") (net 34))
 (segment (start 135.3645 63.7715) (end 136.144 62.992) (width 0.25) (layer "F.Cu") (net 34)))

